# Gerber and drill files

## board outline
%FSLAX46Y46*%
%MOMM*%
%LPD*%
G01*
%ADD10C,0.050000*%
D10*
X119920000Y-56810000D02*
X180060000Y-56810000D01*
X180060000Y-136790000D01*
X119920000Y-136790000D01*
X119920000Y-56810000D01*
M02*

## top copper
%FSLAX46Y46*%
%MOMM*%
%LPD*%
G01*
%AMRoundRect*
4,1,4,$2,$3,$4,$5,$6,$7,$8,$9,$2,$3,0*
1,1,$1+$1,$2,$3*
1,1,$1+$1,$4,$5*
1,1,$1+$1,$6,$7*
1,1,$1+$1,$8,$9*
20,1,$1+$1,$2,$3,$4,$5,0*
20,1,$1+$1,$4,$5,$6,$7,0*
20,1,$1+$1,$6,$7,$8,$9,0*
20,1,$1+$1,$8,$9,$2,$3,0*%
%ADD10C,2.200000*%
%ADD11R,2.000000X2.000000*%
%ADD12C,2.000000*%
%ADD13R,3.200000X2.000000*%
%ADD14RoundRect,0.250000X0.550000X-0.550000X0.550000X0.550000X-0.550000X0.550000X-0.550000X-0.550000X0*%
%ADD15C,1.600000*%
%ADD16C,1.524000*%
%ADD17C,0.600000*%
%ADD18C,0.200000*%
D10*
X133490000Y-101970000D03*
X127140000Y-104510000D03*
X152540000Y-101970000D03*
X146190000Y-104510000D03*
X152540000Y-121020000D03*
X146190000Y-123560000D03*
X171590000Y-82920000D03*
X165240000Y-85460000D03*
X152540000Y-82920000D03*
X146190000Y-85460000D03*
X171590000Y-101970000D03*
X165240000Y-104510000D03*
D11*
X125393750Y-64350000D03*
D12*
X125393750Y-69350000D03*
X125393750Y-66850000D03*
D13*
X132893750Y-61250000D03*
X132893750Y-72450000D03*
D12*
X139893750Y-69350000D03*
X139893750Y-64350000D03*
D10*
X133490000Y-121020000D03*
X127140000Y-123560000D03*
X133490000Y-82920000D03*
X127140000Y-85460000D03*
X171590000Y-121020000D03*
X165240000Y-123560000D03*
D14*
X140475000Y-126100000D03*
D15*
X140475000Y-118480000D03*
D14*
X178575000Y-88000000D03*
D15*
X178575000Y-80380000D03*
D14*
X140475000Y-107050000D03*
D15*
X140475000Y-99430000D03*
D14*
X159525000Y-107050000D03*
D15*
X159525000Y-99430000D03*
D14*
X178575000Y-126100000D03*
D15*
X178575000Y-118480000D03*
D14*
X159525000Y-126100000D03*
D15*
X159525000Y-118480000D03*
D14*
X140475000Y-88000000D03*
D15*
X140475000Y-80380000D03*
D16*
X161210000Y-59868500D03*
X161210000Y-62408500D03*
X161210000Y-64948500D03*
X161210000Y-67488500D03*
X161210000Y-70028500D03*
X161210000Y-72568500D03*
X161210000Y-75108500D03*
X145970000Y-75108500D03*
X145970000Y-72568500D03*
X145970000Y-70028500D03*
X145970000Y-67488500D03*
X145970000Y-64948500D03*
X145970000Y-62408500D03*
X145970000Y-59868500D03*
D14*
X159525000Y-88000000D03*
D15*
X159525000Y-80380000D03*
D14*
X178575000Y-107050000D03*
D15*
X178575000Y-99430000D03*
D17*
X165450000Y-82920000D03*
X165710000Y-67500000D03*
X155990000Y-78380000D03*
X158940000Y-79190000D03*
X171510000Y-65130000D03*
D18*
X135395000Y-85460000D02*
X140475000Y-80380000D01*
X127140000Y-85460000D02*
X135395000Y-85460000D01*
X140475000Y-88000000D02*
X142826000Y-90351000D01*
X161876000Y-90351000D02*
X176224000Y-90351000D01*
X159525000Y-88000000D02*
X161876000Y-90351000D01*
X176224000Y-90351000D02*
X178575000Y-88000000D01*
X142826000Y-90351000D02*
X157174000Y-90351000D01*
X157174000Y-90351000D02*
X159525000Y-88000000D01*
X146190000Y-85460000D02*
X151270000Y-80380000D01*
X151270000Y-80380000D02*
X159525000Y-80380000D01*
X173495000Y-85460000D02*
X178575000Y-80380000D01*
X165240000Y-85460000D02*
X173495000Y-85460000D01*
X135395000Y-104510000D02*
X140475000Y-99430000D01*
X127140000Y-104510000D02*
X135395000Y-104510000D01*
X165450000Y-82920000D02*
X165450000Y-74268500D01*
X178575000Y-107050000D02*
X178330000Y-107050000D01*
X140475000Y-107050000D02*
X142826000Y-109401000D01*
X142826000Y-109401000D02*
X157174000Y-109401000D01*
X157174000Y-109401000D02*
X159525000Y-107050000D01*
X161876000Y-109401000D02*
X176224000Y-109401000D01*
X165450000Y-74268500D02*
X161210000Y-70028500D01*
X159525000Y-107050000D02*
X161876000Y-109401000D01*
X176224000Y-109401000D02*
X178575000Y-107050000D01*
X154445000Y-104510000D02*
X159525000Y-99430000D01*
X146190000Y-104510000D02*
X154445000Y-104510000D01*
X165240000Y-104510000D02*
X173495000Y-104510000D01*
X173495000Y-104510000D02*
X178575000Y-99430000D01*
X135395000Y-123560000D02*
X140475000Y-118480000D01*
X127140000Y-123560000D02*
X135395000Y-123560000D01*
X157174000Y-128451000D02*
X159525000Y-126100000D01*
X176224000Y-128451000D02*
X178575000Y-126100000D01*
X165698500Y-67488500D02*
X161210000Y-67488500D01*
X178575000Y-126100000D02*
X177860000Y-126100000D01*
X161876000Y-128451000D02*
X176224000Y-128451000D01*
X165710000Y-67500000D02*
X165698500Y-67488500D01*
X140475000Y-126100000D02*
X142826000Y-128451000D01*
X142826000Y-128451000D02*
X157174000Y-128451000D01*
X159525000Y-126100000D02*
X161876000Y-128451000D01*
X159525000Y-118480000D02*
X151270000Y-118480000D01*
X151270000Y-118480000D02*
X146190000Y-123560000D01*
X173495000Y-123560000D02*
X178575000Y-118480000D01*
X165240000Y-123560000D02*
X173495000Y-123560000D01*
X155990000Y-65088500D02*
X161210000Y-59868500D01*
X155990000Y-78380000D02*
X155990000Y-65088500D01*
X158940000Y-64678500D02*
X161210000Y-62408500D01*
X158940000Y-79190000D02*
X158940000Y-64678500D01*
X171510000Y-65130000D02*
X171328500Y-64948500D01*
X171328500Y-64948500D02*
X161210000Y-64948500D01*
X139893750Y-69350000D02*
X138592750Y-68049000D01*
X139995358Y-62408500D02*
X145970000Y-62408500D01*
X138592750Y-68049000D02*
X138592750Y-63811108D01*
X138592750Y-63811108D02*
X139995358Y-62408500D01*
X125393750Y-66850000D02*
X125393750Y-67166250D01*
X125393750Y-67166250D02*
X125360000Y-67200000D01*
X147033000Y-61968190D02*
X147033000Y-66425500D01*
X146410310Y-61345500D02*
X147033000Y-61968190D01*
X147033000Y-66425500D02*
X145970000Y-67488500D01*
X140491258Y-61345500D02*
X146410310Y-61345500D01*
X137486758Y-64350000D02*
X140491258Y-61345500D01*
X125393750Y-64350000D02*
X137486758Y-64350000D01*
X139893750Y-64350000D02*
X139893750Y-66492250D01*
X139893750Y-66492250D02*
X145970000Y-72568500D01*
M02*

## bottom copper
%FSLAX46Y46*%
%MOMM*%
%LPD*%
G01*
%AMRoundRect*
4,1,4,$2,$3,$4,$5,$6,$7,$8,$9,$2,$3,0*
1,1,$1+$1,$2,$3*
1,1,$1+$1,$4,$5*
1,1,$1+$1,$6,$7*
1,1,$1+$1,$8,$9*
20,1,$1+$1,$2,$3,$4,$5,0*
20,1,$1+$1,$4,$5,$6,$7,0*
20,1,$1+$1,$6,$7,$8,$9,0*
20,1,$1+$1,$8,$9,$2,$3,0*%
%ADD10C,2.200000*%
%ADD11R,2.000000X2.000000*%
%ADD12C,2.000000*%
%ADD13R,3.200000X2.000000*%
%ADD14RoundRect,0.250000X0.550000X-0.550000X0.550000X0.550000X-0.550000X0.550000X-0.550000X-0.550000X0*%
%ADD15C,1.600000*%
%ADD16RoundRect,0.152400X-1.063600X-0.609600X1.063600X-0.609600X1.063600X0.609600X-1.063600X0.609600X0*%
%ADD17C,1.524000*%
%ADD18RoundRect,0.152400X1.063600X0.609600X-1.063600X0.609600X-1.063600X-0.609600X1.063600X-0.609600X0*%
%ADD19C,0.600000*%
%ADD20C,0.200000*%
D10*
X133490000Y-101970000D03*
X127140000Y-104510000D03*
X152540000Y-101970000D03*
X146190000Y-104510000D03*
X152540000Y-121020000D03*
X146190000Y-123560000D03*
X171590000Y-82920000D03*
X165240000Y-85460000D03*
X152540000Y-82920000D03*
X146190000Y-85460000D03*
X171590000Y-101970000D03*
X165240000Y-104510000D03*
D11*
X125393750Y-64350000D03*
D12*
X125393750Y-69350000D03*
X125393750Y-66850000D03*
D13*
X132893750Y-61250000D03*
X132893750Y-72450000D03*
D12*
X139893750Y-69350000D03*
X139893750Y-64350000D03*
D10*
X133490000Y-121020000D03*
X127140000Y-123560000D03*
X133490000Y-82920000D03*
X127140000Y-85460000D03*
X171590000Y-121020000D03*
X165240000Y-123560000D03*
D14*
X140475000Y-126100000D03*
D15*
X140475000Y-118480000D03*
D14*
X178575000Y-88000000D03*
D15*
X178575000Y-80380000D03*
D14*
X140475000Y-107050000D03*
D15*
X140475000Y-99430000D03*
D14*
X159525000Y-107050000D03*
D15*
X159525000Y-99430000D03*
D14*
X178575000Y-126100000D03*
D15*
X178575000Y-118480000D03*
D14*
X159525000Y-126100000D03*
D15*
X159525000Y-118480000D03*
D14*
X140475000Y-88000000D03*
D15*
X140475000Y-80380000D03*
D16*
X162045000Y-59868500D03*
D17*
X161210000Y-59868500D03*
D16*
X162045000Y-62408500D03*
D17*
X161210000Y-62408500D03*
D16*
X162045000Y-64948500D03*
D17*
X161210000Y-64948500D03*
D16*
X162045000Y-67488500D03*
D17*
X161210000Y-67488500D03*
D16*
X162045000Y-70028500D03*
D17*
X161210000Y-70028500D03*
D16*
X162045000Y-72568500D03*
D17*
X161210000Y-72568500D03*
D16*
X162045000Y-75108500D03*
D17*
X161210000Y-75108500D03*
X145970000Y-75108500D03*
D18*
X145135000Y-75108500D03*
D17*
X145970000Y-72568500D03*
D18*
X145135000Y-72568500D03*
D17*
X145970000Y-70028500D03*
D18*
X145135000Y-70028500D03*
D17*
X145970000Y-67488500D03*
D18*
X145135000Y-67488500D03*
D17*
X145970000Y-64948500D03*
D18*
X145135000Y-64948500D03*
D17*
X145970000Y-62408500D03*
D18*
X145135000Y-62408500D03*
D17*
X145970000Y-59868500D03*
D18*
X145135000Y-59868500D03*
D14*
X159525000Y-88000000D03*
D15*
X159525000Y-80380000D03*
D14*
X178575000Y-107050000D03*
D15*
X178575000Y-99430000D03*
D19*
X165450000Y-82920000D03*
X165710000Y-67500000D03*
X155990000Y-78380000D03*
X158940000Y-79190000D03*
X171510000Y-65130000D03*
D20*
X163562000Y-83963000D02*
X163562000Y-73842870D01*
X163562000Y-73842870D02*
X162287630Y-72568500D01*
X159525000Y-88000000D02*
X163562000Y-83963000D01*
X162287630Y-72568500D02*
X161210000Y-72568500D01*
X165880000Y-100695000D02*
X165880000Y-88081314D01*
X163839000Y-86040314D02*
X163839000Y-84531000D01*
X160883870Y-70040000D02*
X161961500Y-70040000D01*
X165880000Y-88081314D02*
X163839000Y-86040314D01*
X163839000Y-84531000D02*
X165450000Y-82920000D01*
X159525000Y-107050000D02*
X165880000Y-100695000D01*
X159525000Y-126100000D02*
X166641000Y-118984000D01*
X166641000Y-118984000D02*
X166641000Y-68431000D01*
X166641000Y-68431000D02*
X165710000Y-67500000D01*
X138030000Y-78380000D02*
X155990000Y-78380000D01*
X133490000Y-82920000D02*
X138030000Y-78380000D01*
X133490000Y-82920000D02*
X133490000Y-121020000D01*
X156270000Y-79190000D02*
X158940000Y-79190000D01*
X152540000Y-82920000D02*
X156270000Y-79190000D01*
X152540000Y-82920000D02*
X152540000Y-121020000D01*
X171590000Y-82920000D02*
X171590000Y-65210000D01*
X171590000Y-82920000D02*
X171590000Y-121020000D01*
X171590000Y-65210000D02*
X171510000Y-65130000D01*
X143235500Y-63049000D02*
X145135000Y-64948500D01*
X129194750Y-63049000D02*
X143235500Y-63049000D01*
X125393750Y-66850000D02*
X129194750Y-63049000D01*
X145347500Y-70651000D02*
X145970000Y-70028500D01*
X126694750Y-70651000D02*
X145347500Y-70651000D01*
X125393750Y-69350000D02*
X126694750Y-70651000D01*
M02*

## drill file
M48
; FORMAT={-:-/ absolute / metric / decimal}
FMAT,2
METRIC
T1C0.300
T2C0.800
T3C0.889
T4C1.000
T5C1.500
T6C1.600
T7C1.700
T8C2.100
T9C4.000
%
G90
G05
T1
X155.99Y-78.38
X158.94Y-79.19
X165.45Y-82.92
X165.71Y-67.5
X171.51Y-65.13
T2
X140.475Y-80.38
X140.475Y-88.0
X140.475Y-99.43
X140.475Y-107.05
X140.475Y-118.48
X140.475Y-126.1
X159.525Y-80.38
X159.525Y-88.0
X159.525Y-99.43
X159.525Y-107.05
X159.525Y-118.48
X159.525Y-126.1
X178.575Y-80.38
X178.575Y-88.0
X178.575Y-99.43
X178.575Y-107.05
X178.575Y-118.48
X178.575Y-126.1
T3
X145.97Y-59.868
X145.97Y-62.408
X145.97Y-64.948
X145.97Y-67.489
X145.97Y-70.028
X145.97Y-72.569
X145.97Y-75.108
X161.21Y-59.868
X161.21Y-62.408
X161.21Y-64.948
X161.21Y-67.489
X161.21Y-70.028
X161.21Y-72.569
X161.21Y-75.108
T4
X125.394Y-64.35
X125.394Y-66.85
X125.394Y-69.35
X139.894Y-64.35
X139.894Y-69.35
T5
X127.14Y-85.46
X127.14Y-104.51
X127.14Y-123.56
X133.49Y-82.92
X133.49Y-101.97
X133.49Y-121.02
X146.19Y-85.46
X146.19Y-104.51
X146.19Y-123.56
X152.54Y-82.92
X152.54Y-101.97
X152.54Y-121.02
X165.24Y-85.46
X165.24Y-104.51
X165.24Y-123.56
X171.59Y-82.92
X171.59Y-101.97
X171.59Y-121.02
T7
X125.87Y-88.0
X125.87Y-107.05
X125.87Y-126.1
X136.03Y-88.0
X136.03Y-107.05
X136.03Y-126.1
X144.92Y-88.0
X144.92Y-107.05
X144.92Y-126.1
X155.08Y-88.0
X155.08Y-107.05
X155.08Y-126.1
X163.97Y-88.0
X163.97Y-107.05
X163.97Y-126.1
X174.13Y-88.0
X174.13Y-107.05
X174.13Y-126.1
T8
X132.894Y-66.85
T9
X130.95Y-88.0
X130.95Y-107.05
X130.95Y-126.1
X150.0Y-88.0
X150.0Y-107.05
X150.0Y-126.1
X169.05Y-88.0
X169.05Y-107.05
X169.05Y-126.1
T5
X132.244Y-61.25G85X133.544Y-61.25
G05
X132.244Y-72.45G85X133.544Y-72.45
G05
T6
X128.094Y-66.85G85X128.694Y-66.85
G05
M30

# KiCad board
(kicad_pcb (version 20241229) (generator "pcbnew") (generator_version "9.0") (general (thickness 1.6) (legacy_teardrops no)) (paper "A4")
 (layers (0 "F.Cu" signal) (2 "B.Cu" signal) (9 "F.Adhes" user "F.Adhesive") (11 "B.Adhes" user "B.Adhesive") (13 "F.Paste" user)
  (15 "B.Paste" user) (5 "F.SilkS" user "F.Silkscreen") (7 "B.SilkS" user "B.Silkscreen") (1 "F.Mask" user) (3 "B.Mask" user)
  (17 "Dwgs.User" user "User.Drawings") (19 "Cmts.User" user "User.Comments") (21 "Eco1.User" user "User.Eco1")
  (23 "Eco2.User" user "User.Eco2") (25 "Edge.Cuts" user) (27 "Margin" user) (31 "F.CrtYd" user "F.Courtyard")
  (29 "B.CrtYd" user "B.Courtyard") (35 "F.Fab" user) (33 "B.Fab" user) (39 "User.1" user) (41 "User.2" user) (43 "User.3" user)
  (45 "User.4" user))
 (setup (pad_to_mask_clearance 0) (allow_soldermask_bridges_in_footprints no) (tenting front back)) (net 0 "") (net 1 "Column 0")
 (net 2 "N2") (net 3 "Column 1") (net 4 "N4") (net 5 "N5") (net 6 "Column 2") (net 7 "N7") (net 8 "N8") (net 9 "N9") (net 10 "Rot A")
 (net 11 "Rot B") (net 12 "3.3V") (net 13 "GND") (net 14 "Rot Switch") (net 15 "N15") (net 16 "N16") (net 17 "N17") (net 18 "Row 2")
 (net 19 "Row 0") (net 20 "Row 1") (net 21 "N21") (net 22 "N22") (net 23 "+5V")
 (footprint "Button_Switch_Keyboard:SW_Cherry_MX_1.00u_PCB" (layer "F.Cu") (at 133.49 101.97)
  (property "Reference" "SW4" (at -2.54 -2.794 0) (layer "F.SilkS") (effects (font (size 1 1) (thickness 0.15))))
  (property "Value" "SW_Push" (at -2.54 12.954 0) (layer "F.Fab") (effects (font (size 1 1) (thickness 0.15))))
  (pad "" np_thru_hole circle (at -7.62 5.08) (size 1.7 1.7) (drill 1.7) (layers "*.Cu" "*.Mask"))
  (pad "" np_thru_hole circle (at -2.54 5.08) (size 4 4) (drill 4) (layers "*.Cu" "*.Mask"))
  (pad "" np_thru_hole circle (at 2.54 5.08) (size 1.7 1.7) (drill 1.7) (layers "*.Cu" "*.Mask"))
  (pad "1" thru_hole circle (at 0 0) (size 2.2 2.2) (drill 1.5) (layers "*.Cu" "*.Mask") (remove_unused_layers no) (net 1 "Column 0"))
  (pad "2" thru_hole circle (at -6.35 2.54) (size 2.2 2.2) (drill 1.5) (layers "*.Cu" "*.Mask") (remove_unused_layers no) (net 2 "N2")))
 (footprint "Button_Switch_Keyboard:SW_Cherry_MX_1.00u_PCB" (layer "F.Cu") (at 152.54 101.97)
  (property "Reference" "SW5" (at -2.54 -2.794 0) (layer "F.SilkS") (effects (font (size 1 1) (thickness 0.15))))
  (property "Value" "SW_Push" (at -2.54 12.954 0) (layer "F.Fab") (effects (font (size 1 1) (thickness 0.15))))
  (pad "" np_thru_hole circle (at -7.62 5.08) (size 1.7 1.7) (drill 1.7) (layers "*.Cu" "*.Mask"))
  (pad "" np_thru_hole circle (at -2.54 5.08) (size 4 4) (drill 4) (layers "*.Cu" "*.Mask"))
  (pad "" np_thru_hole circle (at 2.54 5.08) (size 1.7 1.7) (drill 1.7) (layers "*.Cu" "*.Mask"))
  (pad "1" thru_hole circle (at 0 0) (size 2.2 2.2) (drill 1.5) (layers "*.Cu" "*.Mask") (remove_unused_layers no) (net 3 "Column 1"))
  (pad "2" thru_hole circle (at -6.35 2.54) (size 2.2 2.2) (drill 1.5) (layers "*.Cu" "*.Mask") (remove_unused_layers no) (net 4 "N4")))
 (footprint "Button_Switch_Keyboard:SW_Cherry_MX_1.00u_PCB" (layer "F.Cu") (at 152.54 121.02)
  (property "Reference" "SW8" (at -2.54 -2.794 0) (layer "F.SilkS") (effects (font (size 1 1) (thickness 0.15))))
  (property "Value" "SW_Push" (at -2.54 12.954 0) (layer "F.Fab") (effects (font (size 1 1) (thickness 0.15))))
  (pad "" np_thru_hole circle (at -7.62 5.08) (size 1.7 1.7) (drill 1.7) (layers "*.Cu" "*.Mask"))
  (pad "" np_thru_hole circle (at -2.54 5.08) (size 4 4) (drill 4) (layers "*.Cu" "*.Mask"))
  (pad "" np_thru_hole circle (at 2.54 5.08) (size 1.7 1.7) (drill 1.7) (layers "*.Cu" "*.Mask"))
  (pad "1" thru_hole circle (at 0 0) (size 2.2 2.2) (drill 1.5) (layers "*.Cu" "*.Mask") (remove_unused_layers no) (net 3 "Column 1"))
  (pad "2" thru_hole circle (at -6.35 2.54) (size 2.2 2.2) (drill 1.5) (layers "*.Cu" "*.Mask") (remove_unused_layers no) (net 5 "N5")))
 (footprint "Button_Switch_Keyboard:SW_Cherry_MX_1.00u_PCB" (layer "F.Cu") (at 171.59 82.92)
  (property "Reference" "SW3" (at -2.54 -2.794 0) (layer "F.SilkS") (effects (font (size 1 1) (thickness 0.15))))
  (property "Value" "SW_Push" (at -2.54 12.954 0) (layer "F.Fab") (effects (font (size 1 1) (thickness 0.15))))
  (pad "" np_thru_hole circle (at -7.62 5.08) (size 1.7 1.7) (drill 1.7) (layers "*.Cu" "*.Mask"))
  (pad "" np_thru_hole circle (at -2.54 5.08) (size 4 4) (drill 4) (layers "*.Cu" "*.Mask"))
  (pad "" np_thru_hole circle (at 2.54 5.08) (size 1.7 1.7) (drill 1.7) (layers "*.Cu" "*.Mask"))
  (pad "1" thru_hole circle (at 0 0) (size 2.2 2.2) (drill 1.5) (layers "*.Cu" "*.Mask") (remove_unused_layers no) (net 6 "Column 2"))
  (pad "2" thru_hole circle (at -6.35 2.54) (size 2.2 2.2) (drill 1.5) (layers "*.Cu" "*.Mask") (remove_unused_layers no) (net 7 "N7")))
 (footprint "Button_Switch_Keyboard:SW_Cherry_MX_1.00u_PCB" (layer "F.Cu") (at 152.54 82.92)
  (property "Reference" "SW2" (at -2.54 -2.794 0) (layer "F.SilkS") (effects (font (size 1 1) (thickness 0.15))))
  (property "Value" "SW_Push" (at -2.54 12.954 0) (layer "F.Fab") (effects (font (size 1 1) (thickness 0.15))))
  (pad "" np_thru_hole circle (at -7.62 5.08) (size 1.7 1.7) (drill 1.7) (layers "*.Cu" "*.Mask"))
  (pad "" np_thru_hole circle (at -2.54 5.08) (size 4 4) (drill 4) (layers "*.Cu" "*.Mask"))
  (pad "" np_thru_hole circle (at 2.54 5.08) (size 1.7 1.7) (drill 1.7) (layers "*.Cu" "*.Mask"))
  (pad "1" thru_hole circle (at 0 0) (size 2.2 2.2) (drill 1.5) (layers "*.Cu" "*.Mask") (remove_unused_layers no) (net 3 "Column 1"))
  (pad "2" thru_hole circle (at -6.35 2.54) (size 2.2 2.2) (drill 1.5) (layers "*.Cu" "*.Mask") (remove_unused_layers no) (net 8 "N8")))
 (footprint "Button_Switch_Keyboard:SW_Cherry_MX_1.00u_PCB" (layer "F.Cu") (at 171.59 101.97)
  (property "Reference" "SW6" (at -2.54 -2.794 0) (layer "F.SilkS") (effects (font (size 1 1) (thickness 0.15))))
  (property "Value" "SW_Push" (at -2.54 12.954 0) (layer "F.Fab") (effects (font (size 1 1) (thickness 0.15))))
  (pad "" np_thru_hole circle (at -7.62 5.08) (size 1.7 1.7) (drill 1.7) (layers "*.Cu" "*.Mask"))
  (pad "" np_thru_hole circle (at -2.54 5.08) (size 4 4) (drill 4) (layers "*.Cu" "*.Mask"))
  (pad "" np_thru_hole circle (at 2.54 5.08) (size 1.7 1.7) (drill 1.7) (layers "*.Cu" "*.Mask"))
  (pad "1" thru_hole circle (at 0 0) (size 2.2 2.2) (drill 1.5) (layers "*.Cu" "*.Mask") (remove_unused_layers no) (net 6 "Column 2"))
  (pad "2" thru_hole circle (at -6.35 2.54) (size 2.2 2.2) (drill 1.5) (layers "*.Cu" "*.Mask") (remove_unused_layers no) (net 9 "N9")))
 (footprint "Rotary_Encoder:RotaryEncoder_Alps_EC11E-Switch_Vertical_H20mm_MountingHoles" (layer "F.Cu") (at 125.39375 64.35)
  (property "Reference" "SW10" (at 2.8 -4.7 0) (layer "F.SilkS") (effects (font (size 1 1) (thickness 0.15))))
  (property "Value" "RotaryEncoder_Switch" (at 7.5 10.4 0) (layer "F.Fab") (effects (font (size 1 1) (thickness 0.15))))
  (pad "" np_thru_hole oval (at 3 2.5) (size 2.2 1.6) (drill oval 2.2 1.6) (layers "*.Mask"))
  (pad "" np_thru_hole circle (at 7.5 2.5) (size 2.1 2.1) (drill 2.1) (layers "*.Mask"))
  (pad "A" thru_hole rect (at 0 0) (size 2 2) (drill 1) (layers "*.Cu" "*.Mask") (remove_unused_layers no) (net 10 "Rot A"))
  (pad "B" thru_hole circle (at 0 5) (size 2 2) (drill 1) (layers "*.Cu" "*.Mask") (remove_unused_layers no) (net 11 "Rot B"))
  (pad "C" thru_hole circle (at 0 2.5) (size 2 2) (drill 1) (layers "*.Cu" "*.Mask") (remove_unused_layers no) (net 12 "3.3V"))
  (pad "MP" thru_hole rect (at 7.5 -3.1) (size 3.2 2) (drill oval 2.8 1.5) (layers "*.Cu" "*.Mask") (remove_unused_layers no))
  (pad "MP" thru_hole rect (at 7.5 8.1) (size 3.2 2) (drill oval 2.8 1.5) (layers "*.Cu" "*.Mask") (remove_unused_layers no))
  (pad "S1" thru_hole circle (at 14.5 5) (size 2 2) (drill 1) (layers "*.Cu" "*.Mask") (remove_unused_layers no) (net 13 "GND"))
  (pad "S2" thru_hole circle (at 14.5 0) (size 2 2) (drill 1) (layers "*.Cu" "*.Mask") (remove_unused_layers no) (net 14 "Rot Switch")))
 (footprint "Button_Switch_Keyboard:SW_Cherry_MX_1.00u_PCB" (layer "F.Cu") (at 133.49 121.02)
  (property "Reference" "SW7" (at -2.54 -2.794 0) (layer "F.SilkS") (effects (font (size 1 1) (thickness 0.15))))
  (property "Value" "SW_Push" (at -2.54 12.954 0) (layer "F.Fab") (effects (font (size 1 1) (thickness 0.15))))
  (pad "" np_thru_hole circle (at -7.62 5.08) (size 1.7 1.7) (drill 1.7) (layers "*.Cu" "*.Mask"))
  (pad "" np_thru_hole circle (at -2.54 5.08) (size 4 4) (drill 4) (layers "*.Cu" "*.Mask"))
  (pad "" np_thru_hole circle (at 2.54 5.08) (size 1.7 1.7) (drill 1.7) (layers "*.Cu" "*.Mask"))
  (pad "1" thru_hole circle (at 0 0) (size 2.2 2.2) (drill 1.5) (layers "*.Cu" "*.Mask") (remove_unused_layers no) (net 1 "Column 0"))
  (pad "2" thru_hole circle (at -6.35 2.54) (size 2.2 2.2) (drill 1.5) (layers "*.Cu" "*.Mask") (remove_unused_layers no) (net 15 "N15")))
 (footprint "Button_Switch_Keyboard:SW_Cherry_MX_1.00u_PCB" (layer "F.Cu") (at 133.49 82.92)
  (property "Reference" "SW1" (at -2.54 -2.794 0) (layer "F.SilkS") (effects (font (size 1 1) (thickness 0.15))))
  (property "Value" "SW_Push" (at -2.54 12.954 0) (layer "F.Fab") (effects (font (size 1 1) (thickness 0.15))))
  (pad "" np_thru_hole circle (at -7.62 5.08) (size 1.7 1.7) (drill 1.7) (layers "*.Cu" "*.Mask"))
  (pad "" np_thru_hole circle (at -2.54 5.08) (size 4 4) (drill 4) (layers "*.Cu" "*.Mask"))
  (pad "" np_thru_hole circle (at 2.54 5.08) (size 1.7 1.7) (drill 1.7) (layers "*.Cu" "*.Mask"))
  (pad "1" thru_hole circle (at 0 0) (size 2.2 2.2) (drill 1.5) (layers "*.Cu" "*.Mask") (remove_unused_layers no) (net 1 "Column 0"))
  (pad "2" thru_hole circle (at -6.35 2.54) (size 2.2 2.2) (drill 1.5) (layers "*.Cu" "*.Mask") (remove_unused_layers no) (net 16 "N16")))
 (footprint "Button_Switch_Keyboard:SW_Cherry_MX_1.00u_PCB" (layer "F.Cu") (at 171.59 121.02)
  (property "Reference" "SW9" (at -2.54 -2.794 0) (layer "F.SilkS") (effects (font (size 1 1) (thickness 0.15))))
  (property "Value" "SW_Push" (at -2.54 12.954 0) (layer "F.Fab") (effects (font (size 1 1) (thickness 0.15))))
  (pad "" np_thru_hole circle (at -7.62 5.08) (size 1.7 1.7) (drill 1.7) (layers "*.Cu" "*.Mask"))
  (pad "" np_thru_hole circle (at -2.54 5.08) (size 4 4) (drill 4) (layers "*.Cu" "*.Mask"))
  (pad "" np_thru_hole circle (at 2.54 5.08) (size 1.7 1.7) (drill 1.7) (layers "*.Cu" "*.Mask"))
  (pad "1" thru_hole circle (at 0 0) (size 2.2 2.2) (drill 1.5) (layers "*.Cu" "*.Mask") (remove_unused_layers no) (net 6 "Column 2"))
  (pad "2" thru_hole circle (at -6.35 2.54) (size 2.2 2.2) (drill 1.5) (layers "*.Cu" "*.Mask") (remove_unused_layers no) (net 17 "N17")))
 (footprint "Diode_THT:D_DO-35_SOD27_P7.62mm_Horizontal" (layer "B.Cu") (at 140.475 126.1 90)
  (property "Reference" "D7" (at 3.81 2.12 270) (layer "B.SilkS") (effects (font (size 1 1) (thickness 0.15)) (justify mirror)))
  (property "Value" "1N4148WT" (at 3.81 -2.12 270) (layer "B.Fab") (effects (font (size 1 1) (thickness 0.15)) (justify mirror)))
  (pad "1" thru_hole roundrect (at 0 0 90) (size 1.6 1.6) (drill 0.8) (layers "*.Cu" "*.Mask") (remove_unused_layers no)
   (roundrect_rratio 0.15625) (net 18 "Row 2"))
  (pad "2" thru_hole circle (at 7.62 0 90) (size 1.6 1.6) (drill 0.8) (layers "*.Cu" "*.Mask") (remove_unused_layers no) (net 15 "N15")))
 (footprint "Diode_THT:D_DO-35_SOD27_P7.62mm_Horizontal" (layer "B.Cu") (at 178.575 88 90)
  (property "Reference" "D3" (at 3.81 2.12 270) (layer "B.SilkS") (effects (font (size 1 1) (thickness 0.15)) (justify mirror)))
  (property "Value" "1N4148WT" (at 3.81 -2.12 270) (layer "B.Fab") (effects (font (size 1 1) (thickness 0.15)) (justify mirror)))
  (pad "1" thru_hole roundrect (at 0 0 90) (size 1.6 1.6) (drill 0.8) (layers "*.Cu" "*.Mask") (remove_unused_layers no)
   (roundrect_rratio 0.15625) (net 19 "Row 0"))
  (pad "2" thru_hole circle (at 7.62 0 90) (size 1.6 1.6) (drill 0.8) (layers "*.Cu" "*.Mask") (remove_unused_layers no) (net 7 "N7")))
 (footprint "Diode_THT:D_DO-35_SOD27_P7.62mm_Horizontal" (layer "B.Cu") (at 140.475 107.05 90)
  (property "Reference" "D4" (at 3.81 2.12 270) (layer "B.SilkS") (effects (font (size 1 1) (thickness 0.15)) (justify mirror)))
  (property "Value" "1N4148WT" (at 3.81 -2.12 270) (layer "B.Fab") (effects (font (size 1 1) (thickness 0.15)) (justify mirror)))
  (pad "1" thru_hole roundrect (at 0 0 90) (size 1.6 1.6) (drill 0.8) (layers "*.Cu" "*.Mask") (remove_unused_layers no)
   (roundrect_rratio 0.15625) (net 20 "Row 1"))
  (pad "2" thru_hole circle (at 7.62 0 90) (size 1.6 1.6) (drill 0.8) (layers "*.Cu" "*.Mask") (remove_unused_layers no) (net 2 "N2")))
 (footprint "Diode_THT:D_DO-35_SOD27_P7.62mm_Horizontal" (layer "B.Cu") (at 159.525 107.05 90)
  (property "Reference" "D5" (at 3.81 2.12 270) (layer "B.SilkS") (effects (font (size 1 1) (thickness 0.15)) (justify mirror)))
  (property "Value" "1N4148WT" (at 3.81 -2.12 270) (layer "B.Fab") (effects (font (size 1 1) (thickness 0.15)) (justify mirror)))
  (pad "1" thru_hole roundrect (at 0 0 90) (size 1.6 1.6) (drill 0.8) (layers "*.Cu" "*.Mask") (remove_unused_layers no)
   (roundrect_rratio 0.15625) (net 20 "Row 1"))
  (pad "2" thru_hole circle (at 7.62 0 90) (size 1.6 1.6) (drill 0.8) (layers "*.Cu" "*.Mask") (remove_unused_layers no) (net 4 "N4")))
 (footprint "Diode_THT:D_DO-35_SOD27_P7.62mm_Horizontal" (layer "B.Cu") (at 178.575 126.1 90)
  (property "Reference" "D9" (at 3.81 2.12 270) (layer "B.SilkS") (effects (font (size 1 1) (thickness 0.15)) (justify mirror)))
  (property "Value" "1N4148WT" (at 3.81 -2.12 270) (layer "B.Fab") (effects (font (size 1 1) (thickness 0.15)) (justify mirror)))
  (pad "1" thru_hole roundrect (at 0 0 90) (size 1.6 1.6) (drill 0.8) (layers "*.Cu" "*.Mask") (remove_unused_layers no)
   (roundrect_rratio 0.15625) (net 18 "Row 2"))
  (pad "2" thru_hole circle (at 7.62 0 90) (size 1.6 1.6) (drill 0.8) (layers "*.Cu" "*.Mask") (remove_unused_layers no) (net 17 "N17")))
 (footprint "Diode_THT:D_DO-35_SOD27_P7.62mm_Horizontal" (layer "B.Cu") (at 159.525 126.1 90)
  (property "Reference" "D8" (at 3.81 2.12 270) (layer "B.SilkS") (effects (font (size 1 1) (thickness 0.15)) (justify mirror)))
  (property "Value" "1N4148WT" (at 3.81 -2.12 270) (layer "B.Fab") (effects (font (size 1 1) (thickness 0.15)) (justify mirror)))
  (pad "1" thru_hole roundrect (at 0 0 90) (size 1.6 1.6) (drill 0.8) (layers "*.Cu" "*.Mask") (remove_unused_layers no)
   (roundrect_rratio 0.15625) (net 18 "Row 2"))
  (pad "2" thru_hole circle (at 7.62 0 90) (size 1.6 1.6) (drill 0.8) (layers "*.Cu" "*.Mask") (remove_unused_layers no) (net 5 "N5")))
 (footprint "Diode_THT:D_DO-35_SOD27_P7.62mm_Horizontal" (layer "B.Cu") (at 140.475 88 90)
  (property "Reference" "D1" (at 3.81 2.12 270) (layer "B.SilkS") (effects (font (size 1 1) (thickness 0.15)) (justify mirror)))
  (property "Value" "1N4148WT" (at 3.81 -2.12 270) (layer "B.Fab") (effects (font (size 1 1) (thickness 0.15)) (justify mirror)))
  (pad "1" thru_hole roundrect (at 0 0 90) (size 1.6 1.6) (drill 0.8) (layers "*.Cu" "*.Mask") (remove_unused_layers no)
   (roundrect_rratio 0.15625) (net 19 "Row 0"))
  (pad "2" thru_hole circle (at 7.62 0 90) (size 1.6 1.6) (drill 0.8) (layers "*.Cu" "*.Mask") (remove_unused_layers no) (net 16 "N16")))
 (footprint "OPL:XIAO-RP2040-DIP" (layer "B.Cu") (at 153.59 67.4885 180)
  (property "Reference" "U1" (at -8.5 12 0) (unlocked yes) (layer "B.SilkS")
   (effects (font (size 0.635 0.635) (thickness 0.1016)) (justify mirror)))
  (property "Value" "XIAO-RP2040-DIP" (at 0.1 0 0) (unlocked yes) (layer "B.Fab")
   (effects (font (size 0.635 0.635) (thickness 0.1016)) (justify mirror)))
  (pad "1" smd roundrect (at -8.455 7.62) (size 2.432 1.524) (layers "B.Cu" "B.Mask") (roundrect_rratio 0.1) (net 1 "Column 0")
   (thermal_bridge_angle 45))
  (pad "1" thru_hole circle (at -7.62 7.62) (size 1.524 1.524) (drill 0.889) (layers "*.Cu" "*.Mask") (remove_unused_layers no)
   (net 1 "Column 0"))
  (pad "2" smd roundrect (at -8.455 5.08) (size 2.432 1.524) (layers "B.Cu" "B.Mask") (roundrect_rratio 0.1) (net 3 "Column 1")
   (thermal_bridge_angle 45))
  (pad "2" thru_hole circle (at -7.62 5.08) (size 1.524 1.524) (drill 0.889) (layers "*.Cu" "*.Mask") (remove_unused_layers no)
   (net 3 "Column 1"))
  (pad "3" smd roundrect (at -8.455 2.54) (size 2.432 1.524) (layers "B.Cu" "B.Mask") (roundrect_rratio 0.1) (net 6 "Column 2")
   (thermal_bridge_angle 45))
  (pad "3" thru_hole circle (at -7.62 2.54) (size 1.524 1.524) (drill 0.889) (layers "*.Cu" "*.Mask") (remove_unused_layers no)
   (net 6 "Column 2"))
  (pad "4" smd roundrect (at -8.455 0) (size 2.432 1.524) (layers "B.Cu" "B.Mask") (roundrect_rratio 0.1) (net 18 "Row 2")
   (thermal_bridge_angle 45))
  (pad "4" thru_hole circle (at -7.62 0) (size 1.524 1.524) (drill 0.889) (layers "*.Cu" "*.Mask") (remove_unused_layers no)
   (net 18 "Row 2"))
  (pad "5" smd roundrect (at -8.455 -2.54) (size 2.432 1.524) (layers "B.Cu" "B.Mask") (roundrect_rratio 0.1) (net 20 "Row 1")
   (thermal_bridge_angle 45))
  (pad "5" thru_hole circle (at -7.62 -2.54) (size 1.524 1.524) (drill 0.889) (layers "*.Cu" "*.Mask") (remove_unused_layers no)
   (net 20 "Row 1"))
  (pad "6" smd roundrect (at -8.455 -5.08) (size 2.432 1.524) (layers "B.Cu" "B.Mask") (roundrect_rratio 0.1) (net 19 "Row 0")
   (thermal_bridge_angle 45))
  (pad "6" thru_hole circle (at -7.62 -5.08) (size 1.524 1.524) (drill 0.889) (layers "*.Cu" "*.Mask") (remove_unused_layers no)
   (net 19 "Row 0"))
  (pad "7" smd roundrect (at -8.455 -7.62) (size 2.432 1.524) (layers "B.Cu" "B.Mask") (roundrect_rratio 0.1) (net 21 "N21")
   (thermal_bridge_angle 45))
  (pad "7" thru_hole circle (at -7.62 -7.62) (size 1.524 1.524) (drill 0.889) (layers "*.Cu" "*.Mask") (remove_unused_layers no)
   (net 21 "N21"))
  (pad "8" thru_hole circle (at 7.62 -7.62 180) (size 1.524 1.524) (drill 0.889) (layers "*.Cu" "*.Mask") (remove_unused_layers no)
   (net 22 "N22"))
  (pad "8" smd roundrect (at 8.455 -7.62 180) (size 2.432 1.524) (layers "B.Cu" "B.Mask") (roundrect_rratio 0.1) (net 22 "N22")
   (thermal_bridge_angle 45))
  (pad "9" thru_hole circle (at 7.62 -5.08 180) (size 1.524 1.524) (drill 0.889) (layers "*.Cu" "*.Mask") (remove_unused_layers no)
   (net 14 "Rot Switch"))
  (pad "9" smd roundrect (at 8.455 -5.08 180) (size 2.432 1.524) (layers "B.Cu" "B.Mask") (roundrect_rratio 0.1) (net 14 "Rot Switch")
   (thermal_bridge_angle 45))
  (pad "10" thru_hole circle (at 7.62 -2.54 180) (size 1.524 1.524) (drill 0.889) (layers "*.Cu" "*.Mask") (remove_unused_layers no)
   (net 11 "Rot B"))
  (pad "10" smd roundrect (at 8.455 -2.54 180) (size 2.432 1.524) (layers "B.Cu" "B.Mask") (roundrect_rratio 0.1) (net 11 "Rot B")
   (thermal_bridge_angle 45))
  (pad "11" thru_hole circle (at 7.62 0 180) (size 1.524 1.524) (drill 0.889) (layers "*.Cu" "*.Mask") (remove_unused_layers no)
   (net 10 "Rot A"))
  (pad "11" smd roundrect (at 8.455 0 180) (size 2.432 1.524) (layers "B.Cu" "B.Mask") (roundrect_rratio 0.1) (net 10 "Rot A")
   (thermal_bridge_angle 45))
  (pad "12" thru_hole circle (at 7.62 2.54 180) (size 1.524 1.524) (drill 0.889) (layers "*.Cu" "*.Mask") (remove_unused_layers no)
   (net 12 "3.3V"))
  (pad "12" smd roundrect (at 8.455 2.54 180) (size 2.432 1.524) (layers "B.Cu" "B.Mask") (roundrect_rratio 0.1) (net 12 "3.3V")
   (thermal_bridge_angle 45))
  (pad "13" thru_hole circle (at 7.62 5.08 180) (size 1.524 1.524) (drill 0.889) (layers "*.Cu" "*.Mask") (remove_unused_layers no)
   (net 13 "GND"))
  (pad "13" smd roundrect (at 8.455 5.08 180) (size 2.432 1.524) (layers "B.Cu" "B.Mask") (roundrect_rratio 0.1) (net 13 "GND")
   (thermal_bridge_angle 45))
  (pad "14" thru_hole circle (at 7.62 7.62 180) (size 1.524 1.524) (drill 0.889) (layers "*.Cu" "*.Mask") (remove_unused_layers no)
   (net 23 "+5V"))
  (pad "14" smd roundrect (at 8.455 7.62 180) (size 2.432 1.524) (layers "B.Cu" "B.Mask") (roundrect_rratio 0.1) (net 23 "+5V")
   (thermal_bridge_angle 45)))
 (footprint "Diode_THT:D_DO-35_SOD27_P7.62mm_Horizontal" (layer "B.Cu") (at 159.525 88 90)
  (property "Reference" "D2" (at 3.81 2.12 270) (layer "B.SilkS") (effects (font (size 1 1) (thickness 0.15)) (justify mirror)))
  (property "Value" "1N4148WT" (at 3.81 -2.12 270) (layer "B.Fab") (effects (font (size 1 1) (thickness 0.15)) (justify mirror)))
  (pad "1" thru_hole roundrect (at 0 0 90) (size 1.6 1.6) (drill 0.8) (layers "*.Cu" "*.Mask") (remove_unused_layers no)
   (roundrect_rratio 0.15625) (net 19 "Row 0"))
  (pad "2" thru_hole circle (at 7.62 0 90) (size 1.6 1.6) (drill 0.8) (layers "*.Cu" "*.Mask") (remove_unused_layers no) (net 8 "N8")))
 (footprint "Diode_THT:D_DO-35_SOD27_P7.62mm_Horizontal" (layer "B.Cu") (at 178.575 107.05 90)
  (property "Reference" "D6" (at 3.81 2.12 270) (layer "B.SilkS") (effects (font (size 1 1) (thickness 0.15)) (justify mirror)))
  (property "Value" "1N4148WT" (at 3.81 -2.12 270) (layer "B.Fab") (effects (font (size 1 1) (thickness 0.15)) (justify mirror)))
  (pad "1" thru_hole roundrect (at 0 0 90) (size 1.6 1.6) (drill 0.8) (layers "*.Cu" "*.Mask") (remove_unused_layers no)
   (roundrect_rratio 0.15625) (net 20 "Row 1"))
  (pad "2" thru_hole circle (at 7.62 0 90) (size 1.6 1.6) (drill 0.8) (layers "*.Cu" "*.Mask") (remove_unused_layers no) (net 9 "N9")))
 (gr_rect (start 119.92 56.81) (end 180.06 136.79) (stroke (width 0.05) (type default)) (fill no) (layer "Edge.Cuts"))
 (segment (start 135.395 85.46) (end 140.475 80.38) (width 0.2) (layer "F.Cu") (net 16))
 (segment (start 127.14 85.46) (end 135.395 85.46) (width 0.2) (layer "F.Cu") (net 16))
 (segment (start 140.475 88) (end 142.826 90.351) (width 0.2) (layer "F.Cu") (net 19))
 (segment (start 161.876 90.351) (end 176.224 90.351) (width 0.2) (layer "F.Cu") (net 19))
 (segment (start 159.525 88) (end 161.876 90.351) (width 0.2) (layer "F.Cu") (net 19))
 (segment (start 176.224 90.351) (end 178.575 88) (width 0.2) (layer "F.Cu") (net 19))
 (segment (start 142.826 90.351) (end 157.174 90.351) (width 0.2) (layer "F.Cu") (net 19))
 (segment (start 157.174 90.351) (end 159.525 88) (width 0.2) (layer "F.Cu") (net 19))
 (segment (start 163.562 83.963) (end 163.562 73.84287) (width 0.2) (layer "B.Cu") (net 19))
 (segment (start 163.562 73.84287) (end 162.28763 72.5685) (width 0.2) (layer "B.Cu") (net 19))
 (segment (start 159.525 88) (end 163.562 83.963) (width 0.2) (layer "B.Cu") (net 19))
 (segment (start 162.28763 72.5685) (end 161.21 72.5685) (width 0.2) (layer "B.Cu") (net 19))
 (segment (start 146.19 85.46) (end 151.27 80.38) (width 0.2) (layer "F.Cu") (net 8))
 (segment (start 151.27 80.38) (end 159.525 80.38) (width 0.2) (layer "F.Cu") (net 8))
 (segment (start 173.495 85.46) (end 178.575 80.38) (width 0.2) (layer "F.Cu") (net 7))
 (segment (start 165.24 85.46) (end 173.495 85.46) (width 0.2) (layer "F.Cu") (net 7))
 (segment (start 135.395 104.51) (end 140.475 99.43) (width 0.2) (layer "F.Cu") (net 2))
 (segment (start 127.14 104.51) (end 135.395 104.51) (width 0.2) (layer "F.Cu") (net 2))
 (segment (start 165.45 82.92) (end 165.45 74.2685) (width 0.2) (layer "F.Cu") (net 20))
 (segment (start 178.575 107.05) (end 178.33 107.05) (width 0.2) (layer "F.Cu") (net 20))
 (segment (start 140.475 107.05) (end 142.826 109.401) (width 0.2) (layer "F.Cu") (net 20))
 (segment (start 142.826 109.401) (end 157.174 109.401) (width 0.2) (layer "F.Cu") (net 20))
 (segment (start 157.174 109.401) (end 159.525 107.05) (width 0.2) (layer "F.Cu") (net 20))
 (segment (start 161.876 109.401) (end 176.224 109.401) (width 0.2) (layer "F.Cu") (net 20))
 (segment (start 165.45 74.2685) (end 161.21 70.0285) (width 0.2) (layer "F.Cu") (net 20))
 (segment (start 159.525 107.05) (end 161.876 109.401) (width 0.2) (layer "F.Cu") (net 20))
 (segment (start 176.224 109.401) (end 178.575 107.05) (width 0.2) (layer "F.Cu") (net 20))
 (via (at 165.45 82.92) (size 0.6) (drill 0.3) (layers "F.Cu" "B.Cu") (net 20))
 (segment (start 165.88 100.695) (end 165.88 88.081314) (width 0.2) (layer "B.Cu") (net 20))
 (segment (start 163.839 86.040314) (end 163.839 84.531) (width 0.2) (layer "B.Cu") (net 20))
 (segment (start 160.88387 70.04) (end 161.9615 70.04) (width 0.2) (layer "B.Cu") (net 20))
 (segment (start 165.88 88.081314) (end 163.839 86.040314) (width 0.2) (layer "B.Cu") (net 20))
 (segment (start 163.839 84.531) (end 165.45 82.92) (width 0.2) (layer "B.Cu") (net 20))
 (segment (start 159.525 107.05) (end 165.88 100.695) (width 0.2) (layer "B.Cu") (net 20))
 (segment (start 154.445 104.51) (end 159.525 99.43) (width 0.2) (layer "F.Cu") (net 4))
 (segment (start 146.19 104.51) (end 154.445 104.51) (width 0.2) (layer "F.Cu") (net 4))
 (segment (start 165.24 104.51) (end 173.495 104.51) (width 0.2) (layer "F.Cu") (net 9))
 (segment (start 173.495 104.51) (end 178.575 99.43) (width 0.2) (layer "F.Cu") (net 9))
 (segment (start 135.395 123.56) (end 140.475 118.48) (width 0.2) (layer "F.Cu") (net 15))
 (segment (start 127.14 123.56) (end 135.395 123.56) (width 0.2) (layer "F.Cu") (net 15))
 (segment (start 157.174 128.451) (end 159.525 126.1) (width 0.2) (layer "F.Cu") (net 18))
 (segment (start 176.224 128.451) (end 178.575 126.1) (width 0.2) (layer "F.Cu") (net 18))
 (segment (start 165.6985 67.4885) (end 161.21 67.4885) (width 0.2) (layer "F.Cu") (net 18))
 (segment (start 178.575 126.1) (end 177.86 126.1) (width 0.2) (layer "F.Cu") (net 18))
 (segment (start 161.876 128.451) (end 176.224 128.451) (width 0.2) (layer "F.Cu") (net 18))
 (segment (start 165.71 67.5) (end 165.6985 67.4885) (width 0.2) (layer "F.Cu") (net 18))
 (segment (start 140.475 126.1) (end 142.826 128.451) (width 0.2) (layer "F.Cu") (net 18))
 (segment (start 142.826 128.451) (end 157.174 128.451) (width 0.2) (layer "F.Cu") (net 18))
 (segment (start 159.525 126.1) (end 161.876 128.451) (width 0.2) (layer "F.Cu") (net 18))
 (via (at 165.71 67.5) (size 0.6) (drill 0.3) (layers "F.Cu" "B.Cu") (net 18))
 (segment (start 159.525 126.1) (end 166.641 118.984) (width 0.2) (layer "B.Cu") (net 18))
 (segment (start 166.641 118.984) (end 166.641 68.431) (width 0.2) (layer "B.Cu") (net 18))
 (segment (start 166.641 68.431) (end 165.71 67.5) (width 0.2) (layer "B.Cu") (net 18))
 (segment (start 159.525 118.48) (end 151.27 118.48) (width 0.2) (layer "F.Cu") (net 5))
 (segment (start 151.27 118.48) (end 146.19 123.56) (width 0.2) (layer "F.Cu") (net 5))
 (segment (start 173.495 123.56) (end 178.575 118.48) (width 0.2) (layer "F.Cu") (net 17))
 (segment (start 165.24 123.56) (end 173.495 123.56) (width 0.2) (layer "F.Cu") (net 17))
 (segment (start 155.99 65.0885) (end 161.21 59.8685) (width 0.2) (layer "F.Cu") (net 1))
 (segment (start 155.99 78.38) (end 155.99 65.0885) (width 0.2) (layer "F.Cu") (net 1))
 (via (at 155.99 78.38) (size 0.6) (drill 0.3) (layers "F.Cu" "B.Cu") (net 1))
 (segment (start 138.03 78.38) (end 155.99 78.38) (width 0.2) (layer "B.Cu") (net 1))
 (segment (start 133.49 82.92) (end 138.03 78.38) (width 0.2) (layer "B.Cu") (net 1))
 (segment (start 133.49 82.92) (end 133.49 121.02) (width 0.2) (layer "B.Cu") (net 1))
 (segment (start 158.94 64.6785) (end 161.21 62.4085) (width 0.2) (layer "F.Cu") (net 3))
 (segment (start 158.94 79.19) (end 158.94 64.6785) (width 0.2) (layer "F.Cu") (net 3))
 (via (at 158.94 79.19) (size 0.6) (drill 0.3) (layers "F.Cu" "B.Cu") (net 3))
 (segment (start 156.27 79.19) (end 158.94 79.19) (width 0.2) (layer "B.Cu") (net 3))
 (segment (start 152.54 82.92) (end 156.27 79.19) (width 0.2) (layer "B.Cu") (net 3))
 (segment (start 152.54 82.92) (end 152.54 121.02) (width 0.2) (layer "B.Cu") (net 3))
 (segment (start 171.51 65.13) (end 171.3285 64.9485) (width 0.2) (layer "F.Cu") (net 6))
 (segment (start 171.3285 64.9485) (end 161.21 64.9485) (width 0.2) (layer "F.Cu") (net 6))
 (via (at 171.51 65.13) (size 0.6) (drill 0.3) (layers "F.Cu" "B.Cu") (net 6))
 (segment (start 171.59 82.92) (end 171.59 65.21) (width 0.2) (layer "B.Cu") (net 6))
 (segment (start 171.59 82.92) (end 171.59 121.02) (width 0.2) (layer "B.Cu") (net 6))
 (segment (start 171.59 65.21) (end 171.51 65.13) (width 0.2) (layer "B.Cu") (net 6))
 (segment (start 139.89375 69.35) (end 138.59275 68.049) (width 0.2) (layer "F.Cu") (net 13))
 (segment (start 139.995358 62.4085) (end 145.97 62.4085) (width 0.2) (layer "F.Cu") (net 13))
 (segment (start 138.59275 68.049) (end 138.59275 63.811108) (width 0.2) (layer "F.Cu") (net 13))
 (segment (start 138.59275 63.811108) (end 139.995358 62.4085) (width 0.2) (layer "F.Cu") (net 13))
 (segment (start 125.39375 66.85) (end 125.39375 67.16625) (width 0.2) (layer "F.Cu") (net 12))
 (segment (start 125.39375 67.16625) (end 125.36 67.2) (width 0.2) (layer "F.Cu") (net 12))
 (segment (start 143.2355 63.049) (end 145.135 64.9485) (width 0.2) (layer "B.Cu") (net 12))
 (segment (start 129.19475 63.049) (end 143.2355 63.049) (width 0.2) (layer "B.Cu") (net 12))
 (segment (start 125.39375 66.85) (end 129.19475 63.049) (width 0.2) (layer "B.Cu") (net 12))
 (segment (start 145.3475 70.651) (end 145.97 70.0285) (width 0.2) (layer "B.Cu") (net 11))
 (segment (start 126.69475 70.651) (end 145.3475 70.651) (width 0.2) (layer "B.Cu") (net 11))
 (segment (start 125.39375 69.35) (end 126.69475 70.651) (width 0.2) (layer "B.Cu") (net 11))
 (segment (start 147.033 61.96819) (end 147.033 66.4255) (width 0.2) (layer "F.Cu") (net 10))
 (segment (start 146.41031 61.3455) (end 147.033 61.96819) (width 0.2) (layer "F.Cu") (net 10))
 (segment (start 147.033 66.4255) (end 145.97 67.4885) (width 0.2) (layer "F.Cu") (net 10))
 (segment (start 140.491258 61.3455) (end 146.41031 61.3455) (width 0.2) (layer "F.Cu") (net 10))
 (segment (start 137.486758 64.35) (end 140.491258 61.3455) (width 0.2) (layer "F.Cu") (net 10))
 (segment (start 125.39375 64.35) (end 137.486758 64.35) (width 0.2) (layer "F.Cu") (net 10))
 (segment (start 139.89375 64.35) (end 139.89375 66.49225) (width 0.2) (layer "F.Cu") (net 14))
 (segment (start 139.89375 66.49225) (end 145.97 72.5685) (width 0.2) (layer "F.Cu") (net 14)))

